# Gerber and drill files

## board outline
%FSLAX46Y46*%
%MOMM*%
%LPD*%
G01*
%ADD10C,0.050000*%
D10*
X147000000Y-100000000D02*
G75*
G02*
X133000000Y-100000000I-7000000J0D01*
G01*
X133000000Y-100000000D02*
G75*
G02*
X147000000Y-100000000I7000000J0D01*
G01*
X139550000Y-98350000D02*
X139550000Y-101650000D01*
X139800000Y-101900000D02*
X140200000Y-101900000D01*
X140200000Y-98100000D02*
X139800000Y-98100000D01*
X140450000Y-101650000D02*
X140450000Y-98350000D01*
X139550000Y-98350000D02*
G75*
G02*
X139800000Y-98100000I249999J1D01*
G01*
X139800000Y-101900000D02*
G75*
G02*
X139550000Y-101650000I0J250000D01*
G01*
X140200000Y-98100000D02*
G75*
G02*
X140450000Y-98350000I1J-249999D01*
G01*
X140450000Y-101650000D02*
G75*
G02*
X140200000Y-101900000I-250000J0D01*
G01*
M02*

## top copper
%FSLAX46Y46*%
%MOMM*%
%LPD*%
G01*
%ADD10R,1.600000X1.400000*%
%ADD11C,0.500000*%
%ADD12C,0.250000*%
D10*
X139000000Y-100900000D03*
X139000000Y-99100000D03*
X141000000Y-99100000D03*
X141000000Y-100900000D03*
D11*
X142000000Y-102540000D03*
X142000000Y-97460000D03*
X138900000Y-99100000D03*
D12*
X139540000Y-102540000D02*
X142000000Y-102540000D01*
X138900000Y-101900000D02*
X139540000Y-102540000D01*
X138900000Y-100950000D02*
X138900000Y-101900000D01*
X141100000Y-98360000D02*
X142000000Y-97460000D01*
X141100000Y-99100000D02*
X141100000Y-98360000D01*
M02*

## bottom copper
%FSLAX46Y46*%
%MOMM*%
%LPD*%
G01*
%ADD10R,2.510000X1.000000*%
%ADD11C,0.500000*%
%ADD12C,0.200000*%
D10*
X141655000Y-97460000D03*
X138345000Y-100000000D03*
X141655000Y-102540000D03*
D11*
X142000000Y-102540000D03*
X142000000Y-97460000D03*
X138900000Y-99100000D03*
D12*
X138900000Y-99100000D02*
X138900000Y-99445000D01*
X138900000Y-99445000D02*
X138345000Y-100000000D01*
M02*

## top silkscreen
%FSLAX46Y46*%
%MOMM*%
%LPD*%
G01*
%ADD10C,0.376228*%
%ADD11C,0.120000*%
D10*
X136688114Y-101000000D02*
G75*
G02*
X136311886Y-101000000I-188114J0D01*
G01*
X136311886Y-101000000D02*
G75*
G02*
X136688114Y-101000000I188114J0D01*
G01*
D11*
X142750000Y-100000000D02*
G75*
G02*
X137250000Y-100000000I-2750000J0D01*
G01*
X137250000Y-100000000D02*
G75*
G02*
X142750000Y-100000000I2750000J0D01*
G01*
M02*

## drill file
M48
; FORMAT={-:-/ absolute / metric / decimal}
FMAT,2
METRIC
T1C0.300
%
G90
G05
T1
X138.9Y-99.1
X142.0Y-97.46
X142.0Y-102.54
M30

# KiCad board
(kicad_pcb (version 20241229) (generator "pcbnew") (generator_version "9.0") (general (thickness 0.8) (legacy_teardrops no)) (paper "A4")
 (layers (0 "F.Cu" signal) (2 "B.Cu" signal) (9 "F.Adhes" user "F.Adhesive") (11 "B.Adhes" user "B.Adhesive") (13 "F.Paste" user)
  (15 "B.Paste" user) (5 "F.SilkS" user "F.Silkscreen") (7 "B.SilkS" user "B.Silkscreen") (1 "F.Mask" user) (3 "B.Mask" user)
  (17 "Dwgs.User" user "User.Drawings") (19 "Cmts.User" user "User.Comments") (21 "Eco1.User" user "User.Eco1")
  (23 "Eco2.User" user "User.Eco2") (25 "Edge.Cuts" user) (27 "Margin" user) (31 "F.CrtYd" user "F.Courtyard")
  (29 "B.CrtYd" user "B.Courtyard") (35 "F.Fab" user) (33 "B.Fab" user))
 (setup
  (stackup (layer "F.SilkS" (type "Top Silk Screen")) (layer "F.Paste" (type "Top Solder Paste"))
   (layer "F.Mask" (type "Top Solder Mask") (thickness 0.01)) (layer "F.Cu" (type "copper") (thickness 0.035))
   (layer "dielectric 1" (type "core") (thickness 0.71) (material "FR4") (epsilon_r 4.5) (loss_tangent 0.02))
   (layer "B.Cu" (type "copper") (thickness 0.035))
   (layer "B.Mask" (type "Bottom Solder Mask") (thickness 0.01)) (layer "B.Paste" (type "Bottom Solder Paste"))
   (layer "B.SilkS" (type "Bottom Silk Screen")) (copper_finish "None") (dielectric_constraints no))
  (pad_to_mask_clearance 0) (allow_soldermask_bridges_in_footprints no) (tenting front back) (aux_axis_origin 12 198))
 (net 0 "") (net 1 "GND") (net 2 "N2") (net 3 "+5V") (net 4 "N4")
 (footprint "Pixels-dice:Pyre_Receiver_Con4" (layer "F.Cu") (at 140 100 -90)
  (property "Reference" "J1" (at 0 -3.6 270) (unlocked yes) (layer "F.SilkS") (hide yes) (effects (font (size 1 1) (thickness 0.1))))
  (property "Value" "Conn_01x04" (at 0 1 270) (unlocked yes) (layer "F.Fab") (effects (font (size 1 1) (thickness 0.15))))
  (fp_line (start -1.65 0.45) (end 1.65 0.45) (stroke (width 0.05) (type default)) (layer "Edge.Cuts"))
  (fp_line (start 1.9 0.2) (end 1.9 -0.2) (stroke (width 0.05) (type solid)) (layer "Edge.Cuts"))
  (fp_line (start -1.9 -0.2) (end -1.9 0.2) (stroke (width 0.05) (type default)) (layer "Edge.Cuts"))
  (fp_line (start 1.65 -0.45) (end -1.65 -0.45) (stroke (width 0.05) (type default)) (layer "Edge.Cuts"))
  (fp_arc (start -1.65 0.45) (mid -1.826777 0.376777) (end -1.9 0.2) (stroke (width 0.05) (type default)) (layer "Edge.Cuts"))
  (fp_arc (start 1.9 0.2) (mid 1.826777 0.376778) (end 1.65 0.45) (stroke (width 0.05) (type default)) (layer "Edge.Cuts"))
  (fp_arc (start -1.9 -0.2) (mid -1.826777 -0.376777) (end -1.65 -0.45) (stroke (width 0.05) (type default)) (layer "Edge.Cuts"))
  (fp_arc (start 1.65 -0.45) (mid 1.826775 -0.376776) (end 1.9 -0.2) (stroke (width 0.05) (type default)) (layer "Edge.Cuts"))
  (pad "1" connect rect (at 0.9 1 270) (size 1.4 1.6) (layers "F.Cu" "F.Mask") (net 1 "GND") (thermal_bridge_angle 45))
  (pad "2" connect rect (at -0.9 1 270) (size 1.4 1.6) (layers "F.Cu" "F.Mask") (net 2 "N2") (thermal_bridge_angle 45))
  (pad "3" connect rect (at -0.9 -1 270) (size 1.4 1.6) (layers "F.Cu" "F.Mask") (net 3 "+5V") (thermal_bridge_angle 45))
  (pad "4" connect rect (at 0.9 -1 270) (size 1.4 1.6) (layers "F.Cu" "F.Mask") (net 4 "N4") (thermal_bridge_angle 45)))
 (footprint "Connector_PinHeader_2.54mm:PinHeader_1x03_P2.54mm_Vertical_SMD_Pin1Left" (layer "B.Cu") (at 140 100 180)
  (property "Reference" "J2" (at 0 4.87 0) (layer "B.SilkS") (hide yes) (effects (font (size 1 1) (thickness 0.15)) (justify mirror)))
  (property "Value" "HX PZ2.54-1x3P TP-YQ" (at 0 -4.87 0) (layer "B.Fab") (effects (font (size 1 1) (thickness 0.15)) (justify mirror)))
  (pad "1" smd rect (at -1.655 2.54 180) (size 2.51 1) (layers "B.Cu" "B.Mask" "B.Paste") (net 3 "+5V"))
  (pad "2" smd rect (at 1.655 0 180) (size 2.51 1) (layers "B.Cu" "B.Mask" "B.Paste") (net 2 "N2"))
  (pad "3" smd rect (at -1.655 -2.54 180) (size 2.51 1) (layers "B.Cu" "B.Mask" "B.Paste") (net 1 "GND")))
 (gr_circle (center 136.5 101) (end 136.8 101.1) (stroke (width 0.12) (type solid)) (fill yes) (layer "F.SilkS"))
 (gr_circle (center 140 100) (end 142.75 100) (stroke (width 0.12) (type default)) (fill no) (layer "F.SilkS"))
 (gr_circle (center 140 100) (end 147 100) (stroke (width 0.05) (type solid)) (fill no) (layer "Edge.Cuts"))
 (segment (start 139.54 102.54) (end 142 102.54) (width 0.25) (layer "F.Cu") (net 1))
 (segment (start 138.9 101.9) (end 139.54 102.54) (width 0.25) (layer "F.Cu") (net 1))
 (segment (start 138.9 100.95) (end 138.9 101.9) (width 0.25) (layer "F.Cu") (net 1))
 (via (at 142 102.54) (size 0.5) (drill 0.3) (layers "F.Cu" "B.Cu") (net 1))
 (segment (start 141.1 98.36) (end 142 97.46) (width 0.25) (layer "F.Cu") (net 3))
 (segment (start 141.1 99.1) (end 141.1 98.36) (width 0.25) (layer "F.Cu") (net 3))
 (via (at 142 97.46) (size 0.5) (drill 0.3) (layers "F.Cu" "B.Cu") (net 3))
 (via (at 138.9 99.1) (size 0.5) (drill 0.3) (layers "F.Cu" "B.Cu") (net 2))
 (segment (start 138.9 99.1) (end 138.9 99.445) (width 0.2) (layer "B.Cu") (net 2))
 (segment (start 138.9 99.445) (end 138.345 100) (width 0.2) (layer "B.Cu") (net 2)))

